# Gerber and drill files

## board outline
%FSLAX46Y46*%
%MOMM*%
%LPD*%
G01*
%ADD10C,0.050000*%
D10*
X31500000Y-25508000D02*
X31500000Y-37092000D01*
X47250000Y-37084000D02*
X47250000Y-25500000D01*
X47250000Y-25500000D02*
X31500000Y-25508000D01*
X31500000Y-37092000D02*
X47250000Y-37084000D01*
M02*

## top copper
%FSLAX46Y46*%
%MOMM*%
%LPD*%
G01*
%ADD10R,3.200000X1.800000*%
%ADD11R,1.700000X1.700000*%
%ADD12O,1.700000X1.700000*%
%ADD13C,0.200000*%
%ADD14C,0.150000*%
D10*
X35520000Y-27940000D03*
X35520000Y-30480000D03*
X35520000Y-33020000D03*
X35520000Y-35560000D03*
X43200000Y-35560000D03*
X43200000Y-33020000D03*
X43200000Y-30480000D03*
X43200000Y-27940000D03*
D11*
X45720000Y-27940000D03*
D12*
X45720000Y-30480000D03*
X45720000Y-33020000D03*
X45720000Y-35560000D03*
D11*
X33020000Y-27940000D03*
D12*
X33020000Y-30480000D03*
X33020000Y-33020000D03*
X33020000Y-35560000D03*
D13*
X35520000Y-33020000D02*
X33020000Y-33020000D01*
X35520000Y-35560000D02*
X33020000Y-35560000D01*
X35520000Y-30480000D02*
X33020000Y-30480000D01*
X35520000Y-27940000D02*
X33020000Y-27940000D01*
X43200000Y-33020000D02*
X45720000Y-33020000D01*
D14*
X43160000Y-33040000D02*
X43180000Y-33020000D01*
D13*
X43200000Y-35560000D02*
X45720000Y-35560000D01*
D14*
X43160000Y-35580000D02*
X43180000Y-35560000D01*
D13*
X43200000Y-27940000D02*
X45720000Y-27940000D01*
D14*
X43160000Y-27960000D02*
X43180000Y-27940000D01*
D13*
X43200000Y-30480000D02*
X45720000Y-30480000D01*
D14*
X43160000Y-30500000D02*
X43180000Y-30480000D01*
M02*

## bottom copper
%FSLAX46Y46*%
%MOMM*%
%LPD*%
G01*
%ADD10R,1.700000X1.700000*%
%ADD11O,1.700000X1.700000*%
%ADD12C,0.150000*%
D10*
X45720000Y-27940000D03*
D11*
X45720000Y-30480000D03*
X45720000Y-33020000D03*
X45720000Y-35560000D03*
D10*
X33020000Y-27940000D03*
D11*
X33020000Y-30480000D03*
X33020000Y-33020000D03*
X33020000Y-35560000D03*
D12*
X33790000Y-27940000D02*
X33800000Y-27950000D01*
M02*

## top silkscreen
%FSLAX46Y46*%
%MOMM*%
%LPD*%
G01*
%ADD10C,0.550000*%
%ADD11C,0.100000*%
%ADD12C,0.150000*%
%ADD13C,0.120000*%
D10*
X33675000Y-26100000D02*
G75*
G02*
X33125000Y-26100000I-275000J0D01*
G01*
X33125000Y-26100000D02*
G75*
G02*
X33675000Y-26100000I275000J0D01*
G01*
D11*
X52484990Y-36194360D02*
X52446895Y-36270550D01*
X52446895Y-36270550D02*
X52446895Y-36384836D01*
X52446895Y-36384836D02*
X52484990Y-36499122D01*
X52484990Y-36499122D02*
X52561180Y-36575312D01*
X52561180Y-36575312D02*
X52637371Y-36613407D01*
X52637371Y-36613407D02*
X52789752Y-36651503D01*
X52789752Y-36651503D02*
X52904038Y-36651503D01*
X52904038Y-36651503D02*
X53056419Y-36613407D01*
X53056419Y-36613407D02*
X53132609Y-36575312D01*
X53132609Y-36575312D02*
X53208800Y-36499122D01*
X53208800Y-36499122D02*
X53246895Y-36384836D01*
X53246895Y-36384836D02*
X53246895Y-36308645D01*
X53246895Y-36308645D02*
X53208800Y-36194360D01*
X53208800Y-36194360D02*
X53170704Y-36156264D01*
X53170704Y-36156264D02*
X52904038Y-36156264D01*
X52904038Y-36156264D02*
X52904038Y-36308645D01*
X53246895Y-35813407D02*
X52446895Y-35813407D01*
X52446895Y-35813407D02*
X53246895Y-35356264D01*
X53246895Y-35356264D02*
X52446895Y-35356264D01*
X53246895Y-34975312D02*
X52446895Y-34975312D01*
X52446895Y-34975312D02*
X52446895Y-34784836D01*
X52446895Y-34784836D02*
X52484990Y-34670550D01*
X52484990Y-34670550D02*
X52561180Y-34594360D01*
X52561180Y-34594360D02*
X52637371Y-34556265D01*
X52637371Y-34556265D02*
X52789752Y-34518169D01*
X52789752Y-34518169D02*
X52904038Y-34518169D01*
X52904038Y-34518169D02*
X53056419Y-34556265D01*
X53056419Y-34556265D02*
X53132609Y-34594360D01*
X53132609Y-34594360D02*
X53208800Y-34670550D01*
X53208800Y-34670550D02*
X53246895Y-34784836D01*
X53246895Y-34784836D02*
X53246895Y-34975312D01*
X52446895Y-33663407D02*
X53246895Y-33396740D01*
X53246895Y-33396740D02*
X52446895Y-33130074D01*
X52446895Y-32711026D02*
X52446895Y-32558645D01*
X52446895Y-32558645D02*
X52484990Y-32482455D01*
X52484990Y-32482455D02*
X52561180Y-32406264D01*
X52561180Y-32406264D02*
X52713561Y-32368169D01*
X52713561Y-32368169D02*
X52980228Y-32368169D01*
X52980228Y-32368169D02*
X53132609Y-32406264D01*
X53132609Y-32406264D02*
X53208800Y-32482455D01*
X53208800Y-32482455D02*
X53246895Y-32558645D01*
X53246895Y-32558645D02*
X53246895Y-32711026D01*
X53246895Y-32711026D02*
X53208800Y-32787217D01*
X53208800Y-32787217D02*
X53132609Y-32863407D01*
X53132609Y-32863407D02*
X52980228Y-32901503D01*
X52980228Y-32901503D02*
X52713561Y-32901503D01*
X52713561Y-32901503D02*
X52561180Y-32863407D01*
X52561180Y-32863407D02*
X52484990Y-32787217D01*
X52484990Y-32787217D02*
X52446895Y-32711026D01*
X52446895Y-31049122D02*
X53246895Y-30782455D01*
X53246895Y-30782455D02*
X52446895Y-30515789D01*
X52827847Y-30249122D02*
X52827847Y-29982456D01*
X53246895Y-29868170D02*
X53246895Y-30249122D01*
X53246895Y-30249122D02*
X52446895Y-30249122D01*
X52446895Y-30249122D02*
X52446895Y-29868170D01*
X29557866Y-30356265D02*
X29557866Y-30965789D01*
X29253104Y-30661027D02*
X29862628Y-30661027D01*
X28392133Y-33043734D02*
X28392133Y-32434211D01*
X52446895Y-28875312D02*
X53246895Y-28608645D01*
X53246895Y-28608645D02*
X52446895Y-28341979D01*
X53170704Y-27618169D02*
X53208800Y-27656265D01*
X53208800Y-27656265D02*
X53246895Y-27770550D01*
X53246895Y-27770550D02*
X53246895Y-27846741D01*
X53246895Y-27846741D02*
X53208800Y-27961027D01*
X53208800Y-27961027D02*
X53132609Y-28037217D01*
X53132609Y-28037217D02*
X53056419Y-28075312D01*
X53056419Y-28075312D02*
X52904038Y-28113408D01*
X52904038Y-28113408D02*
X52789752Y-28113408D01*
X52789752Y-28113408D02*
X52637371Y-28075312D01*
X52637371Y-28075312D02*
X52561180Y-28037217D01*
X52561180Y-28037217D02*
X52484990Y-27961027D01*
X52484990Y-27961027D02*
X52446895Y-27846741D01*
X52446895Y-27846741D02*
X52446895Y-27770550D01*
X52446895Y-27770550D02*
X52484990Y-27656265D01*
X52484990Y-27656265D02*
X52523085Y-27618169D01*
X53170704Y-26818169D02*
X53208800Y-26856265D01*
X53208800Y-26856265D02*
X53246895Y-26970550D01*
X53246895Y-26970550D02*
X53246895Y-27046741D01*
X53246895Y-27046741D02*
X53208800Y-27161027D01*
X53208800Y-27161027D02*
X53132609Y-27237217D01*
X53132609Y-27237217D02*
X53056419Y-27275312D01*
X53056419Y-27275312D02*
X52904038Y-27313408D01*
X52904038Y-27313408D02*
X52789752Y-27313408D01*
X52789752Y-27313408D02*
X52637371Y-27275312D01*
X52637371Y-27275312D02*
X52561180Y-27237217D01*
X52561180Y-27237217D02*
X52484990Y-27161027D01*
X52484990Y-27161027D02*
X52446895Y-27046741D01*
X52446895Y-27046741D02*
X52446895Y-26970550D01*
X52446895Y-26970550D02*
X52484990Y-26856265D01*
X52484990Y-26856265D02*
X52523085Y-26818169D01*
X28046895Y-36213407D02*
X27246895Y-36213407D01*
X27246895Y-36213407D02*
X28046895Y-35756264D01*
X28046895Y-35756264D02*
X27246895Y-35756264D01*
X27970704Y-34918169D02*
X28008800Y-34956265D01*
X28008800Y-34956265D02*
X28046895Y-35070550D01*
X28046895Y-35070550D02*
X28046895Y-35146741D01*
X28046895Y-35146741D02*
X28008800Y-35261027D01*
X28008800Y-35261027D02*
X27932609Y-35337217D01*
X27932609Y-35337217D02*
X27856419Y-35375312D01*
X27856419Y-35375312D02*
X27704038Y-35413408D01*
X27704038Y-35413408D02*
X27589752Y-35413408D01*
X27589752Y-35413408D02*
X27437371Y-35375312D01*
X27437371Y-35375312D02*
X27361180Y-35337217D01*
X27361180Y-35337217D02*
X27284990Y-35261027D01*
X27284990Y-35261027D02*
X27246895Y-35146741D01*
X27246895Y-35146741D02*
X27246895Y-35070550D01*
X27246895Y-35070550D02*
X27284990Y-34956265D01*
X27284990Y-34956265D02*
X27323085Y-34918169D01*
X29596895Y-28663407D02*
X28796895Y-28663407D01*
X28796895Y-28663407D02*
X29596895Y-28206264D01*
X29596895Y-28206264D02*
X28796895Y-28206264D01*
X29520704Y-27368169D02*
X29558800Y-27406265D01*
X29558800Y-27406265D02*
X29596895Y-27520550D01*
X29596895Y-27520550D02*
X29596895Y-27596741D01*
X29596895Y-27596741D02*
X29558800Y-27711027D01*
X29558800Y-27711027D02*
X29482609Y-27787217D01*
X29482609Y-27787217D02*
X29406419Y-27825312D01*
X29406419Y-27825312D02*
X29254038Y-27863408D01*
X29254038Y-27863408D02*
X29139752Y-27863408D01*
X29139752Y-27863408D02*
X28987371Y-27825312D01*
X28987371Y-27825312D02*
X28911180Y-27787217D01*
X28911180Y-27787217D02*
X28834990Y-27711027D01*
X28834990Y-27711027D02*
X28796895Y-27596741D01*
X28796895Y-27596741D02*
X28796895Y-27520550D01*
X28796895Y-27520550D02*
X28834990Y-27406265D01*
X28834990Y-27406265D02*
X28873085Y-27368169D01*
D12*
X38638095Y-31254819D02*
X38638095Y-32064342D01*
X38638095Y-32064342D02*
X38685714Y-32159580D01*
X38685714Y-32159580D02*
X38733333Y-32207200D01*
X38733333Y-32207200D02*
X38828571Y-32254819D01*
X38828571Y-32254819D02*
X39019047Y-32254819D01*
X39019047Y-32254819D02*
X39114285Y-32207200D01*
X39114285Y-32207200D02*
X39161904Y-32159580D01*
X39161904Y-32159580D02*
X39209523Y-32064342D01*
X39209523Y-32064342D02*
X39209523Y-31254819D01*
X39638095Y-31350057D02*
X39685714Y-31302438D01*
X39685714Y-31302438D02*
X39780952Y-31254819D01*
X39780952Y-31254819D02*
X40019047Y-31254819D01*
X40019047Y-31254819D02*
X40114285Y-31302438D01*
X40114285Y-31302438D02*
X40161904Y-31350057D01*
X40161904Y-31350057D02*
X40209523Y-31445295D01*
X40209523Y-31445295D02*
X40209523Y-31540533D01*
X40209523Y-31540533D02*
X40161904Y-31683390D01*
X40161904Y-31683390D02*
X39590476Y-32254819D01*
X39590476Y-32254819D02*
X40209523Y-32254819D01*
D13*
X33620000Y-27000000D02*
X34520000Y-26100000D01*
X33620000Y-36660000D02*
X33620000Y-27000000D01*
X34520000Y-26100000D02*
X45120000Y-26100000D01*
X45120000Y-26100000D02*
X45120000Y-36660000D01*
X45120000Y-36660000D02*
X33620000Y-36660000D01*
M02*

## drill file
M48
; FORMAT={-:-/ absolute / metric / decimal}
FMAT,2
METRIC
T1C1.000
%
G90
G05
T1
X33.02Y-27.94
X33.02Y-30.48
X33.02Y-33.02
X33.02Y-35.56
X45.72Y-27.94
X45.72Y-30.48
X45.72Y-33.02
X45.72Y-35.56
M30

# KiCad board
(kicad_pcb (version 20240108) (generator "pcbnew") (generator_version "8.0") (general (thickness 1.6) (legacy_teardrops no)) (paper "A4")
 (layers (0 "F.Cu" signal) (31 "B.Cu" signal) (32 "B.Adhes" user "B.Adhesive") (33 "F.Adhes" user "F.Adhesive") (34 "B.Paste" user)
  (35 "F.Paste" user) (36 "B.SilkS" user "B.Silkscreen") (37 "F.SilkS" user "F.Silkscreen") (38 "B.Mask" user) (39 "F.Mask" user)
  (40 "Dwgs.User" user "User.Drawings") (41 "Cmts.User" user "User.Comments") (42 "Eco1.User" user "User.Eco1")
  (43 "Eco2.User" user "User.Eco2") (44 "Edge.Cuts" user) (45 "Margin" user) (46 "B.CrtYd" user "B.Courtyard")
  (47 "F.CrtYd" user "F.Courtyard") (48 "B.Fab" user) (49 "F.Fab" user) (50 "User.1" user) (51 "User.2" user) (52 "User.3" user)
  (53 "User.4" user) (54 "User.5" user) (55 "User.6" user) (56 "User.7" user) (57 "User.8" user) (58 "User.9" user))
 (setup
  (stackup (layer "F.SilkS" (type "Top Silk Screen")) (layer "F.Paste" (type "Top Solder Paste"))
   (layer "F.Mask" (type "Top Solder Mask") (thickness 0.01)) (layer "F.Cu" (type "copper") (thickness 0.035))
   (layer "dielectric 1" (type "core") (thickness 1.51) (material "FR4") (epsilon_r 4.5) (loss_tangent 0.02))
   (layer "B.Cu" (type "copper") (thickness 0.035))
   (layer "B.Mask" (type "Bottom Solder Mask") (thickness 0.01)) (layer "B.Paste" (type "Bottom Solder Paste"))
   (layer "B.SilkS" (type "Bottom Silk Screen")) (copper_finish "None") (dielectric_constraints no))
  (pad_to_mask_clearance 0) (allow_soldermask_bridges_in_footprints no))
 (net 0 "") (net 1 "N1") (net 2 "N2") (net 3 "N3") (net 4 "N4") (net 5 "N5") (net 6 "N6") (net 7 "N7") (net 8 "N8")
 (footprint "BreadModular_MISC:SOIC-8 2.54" (layer "F.Cu") (at 38.12 31.75 -90)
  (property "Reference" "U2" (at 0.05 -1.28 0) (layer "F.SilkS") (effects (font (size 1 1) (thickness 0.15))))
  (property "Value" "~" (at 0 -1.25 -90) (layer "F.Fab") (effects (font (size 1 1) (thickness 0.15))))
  (fp_line (start -4.75 4.5) (end -5.65 3.6) (stroke (width 0.12) (type default)) (layer "F.SilkS"))
  (fp_line (start 4.91 4.5) (end -4.75 4.5) (stroke (width 0.12) (type default)) (layer "F.SilkS"))
  (fp_line (start -5.65 3.6) (end -5.65 -7) (stroke (width 0.12) (type default)) (layer "F.SilkS"))
  (fp_line (start -5.65 -7) (end 4.91 -7) (stroke (width 0.12) (type default)) (layer "F.SilkS"))
  (fp_line (start 4.91 -7) (end 4.91 4.5) (stroke (width 0.12) (type default)) (layer "F.SilkS"))
  (pad "1" smd rect (at -3.81 2.6 270) (size 1.8 3.2) (layers "F.Cu" "F.Paste" "F.Mask") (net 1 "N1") (thermal_bridge_angle 45))
  (pad "2" smd rect (at -1.27 2.6 270) (size 1.8 3.2) (layers "F.Cu" "F.Paste" "F.Mask") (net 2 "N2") (thermal_bridge_angle 45))
  (pad "3" smd rect (at 1.27 2.6 270) (size 1.8 3.2) (layers "F.Cu" "F.Paste" "F.Mask") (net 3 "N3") (thermal_bridge_angle 45))
  (pad "4" smd rect (at 3.81 2.6 270) (size 1.8 3.2) (layers "F.Cu" "F.Paste" "F.Mask") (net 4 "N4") (thermal_bridge_angle 45))
  (pad "5" smd rect (at 3.81 -5.08 270) (size 1.8 3.2) (layers "F.Cu" "F.Paste" "F.Mask") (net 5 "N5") (thermal_bridge_angle 45))
  (pad "6" smd rect (at 1.27 -5.08 270) (size 1.8 3.2) (layers "F.Cu" "F.Paste" "F.Mask") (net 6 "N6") (thermal_bridge_angle 45))
  (pad "7" smd rect (at -1.27 -5.08 270) (size 1.8 3.2) (layers "F.Cu" "F.Paste" "F.Mask") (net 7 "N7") (thermal_bridge_angle 45))
  (pad "8" smd rect (at -3.81 -5.08 270) (size 1.8 3.2) (layers "F.Cu" "F.Paste" "F.Mask") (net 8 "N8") (thermal_bridge_angle 45)))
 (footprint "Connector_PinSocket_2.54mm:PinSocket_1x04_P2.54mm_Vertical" (layer "B.Cu") (at 45.72 27.94 180)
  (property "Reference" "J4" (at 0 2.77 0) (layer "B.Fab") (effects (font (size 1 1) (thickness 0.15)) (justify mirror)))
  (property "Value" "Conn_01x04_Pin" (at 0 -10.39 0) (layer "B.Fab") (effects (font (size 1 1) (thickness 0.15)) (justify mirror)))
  (pad "1" thru_hole rect (at 0 0 180) (size 1.7 1.7) (drill 1) (layers "*.Cu" "*.Mask") (remove_unused_layers no) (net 8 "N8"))
  (pad "2" thru_hole oval (at 0 -2.54 180) (size 1.7 1.7) (drill 1) (layers "*.Cu" "*.Mask") (remove_unused_layers no) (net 7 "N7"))
  (pad "3" thru_hole oval (at 0 -5.08 180) (size 1.7 1.7) (drill 1) (layers "*.Cu" "*.Mask") (remove_unused_layers no) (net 6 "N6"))
  (pad "4" thru_hole oval (at 0 -7.62 180) (size 1.7 1.7) (drill 1) (layers "*.Cu" "*.Mask") (remove_unused_layers no) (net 5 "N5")))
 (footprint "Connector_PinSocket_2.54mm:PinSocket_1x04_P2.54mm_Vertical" (layer "B.Cu") (at 33.02 27.94 180)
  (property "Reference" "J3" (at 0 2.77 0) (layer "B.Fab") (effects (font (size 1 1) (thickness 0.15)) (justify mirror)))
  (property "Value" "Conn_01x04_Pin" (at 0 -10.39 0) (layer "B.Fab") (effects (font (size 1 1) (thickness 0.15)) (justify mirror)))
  (pad "1" thru_hole rect (at 0 0 180) (size 1.7 1.7) (drill 1) (layers "*.Cu" "*.Mask") (remove_unused_layers no) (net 1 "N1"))
  (pad "2" thru_hole oval (at 0 -2.54 180) (size 1.7 1.7) (drill 1) (layers "*.Cu" "*.Mask") (remove_unused_layers no) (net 2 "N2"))
  (pad "3" thru_hole oval (at 0 -5.08 180) (size 1.7 1.7) (drill 1) (layers "*.Cu" "*.Mask") (remove_unused_layers no) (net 3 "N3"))
  (pad "4" thru_hole oval (at 0 -7.62 180) (size 1.7 1.7) (drill 1) (layers "*.Cu" "*.Mask") (remove_unused_layers no) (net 4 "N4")))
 (gr_circle (center 33.4 26.1) (end 33.9 26.1) (stroke (width 0.1) (type solid)) (fill solid) (layer "F.SilkS"))
 (gr_line (start 31.5 25.508) (end 31.5 37.092) (stroke (width 0.05) (type default)) (layer "Edge.Cuts"))
 (gr_line (start 47.25 37.084) (end 47.25 25.5) (stroke (width 0.05) (type default)) (layer "Edge.Cuts"))
 (gr_line (start 47.25 25.5) (end 31.5 25.508) (stroke (width 0.05) (type default)) (layer "Edge.Cuts"))
 (gr_line (start 31.5 37.092) (end 47.25 37.084) (stroke (width 0.05) (type default)) (layer "Edge.Cuts"))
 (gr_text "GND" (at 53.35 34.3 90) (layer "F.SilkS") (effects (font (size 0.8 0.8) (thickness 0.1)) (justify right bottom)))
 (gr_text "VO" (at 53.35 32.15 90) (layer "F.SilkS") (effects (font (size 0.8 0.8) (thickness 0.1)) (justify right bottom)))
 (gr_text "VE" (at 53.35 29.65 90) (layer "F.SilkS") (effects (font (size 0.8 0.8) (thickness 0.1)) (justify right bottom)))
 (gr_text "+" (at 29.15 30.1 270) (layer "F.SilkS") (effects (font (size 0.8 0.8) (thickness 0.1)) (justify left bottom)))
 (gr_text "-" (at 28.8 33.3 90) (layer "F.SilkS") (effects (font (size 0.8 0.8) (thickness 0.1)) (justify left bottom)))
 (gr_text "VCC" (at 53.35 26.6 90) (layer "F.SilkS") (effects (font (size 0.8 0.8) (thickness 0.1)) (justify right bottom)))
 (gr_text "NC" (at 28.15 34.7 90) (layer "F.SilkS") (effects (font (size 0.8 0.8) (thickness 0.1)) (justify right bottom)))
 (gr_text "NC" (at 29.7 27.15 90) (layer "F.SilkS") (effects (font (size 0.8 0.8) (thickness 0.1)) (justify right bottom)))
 (segment (start 35.52 33.02) (end 33.02 33.02) (width 0.2) (layer "F.Cu") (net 3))
 (segment (start 35.52 35.56) (end 33.02 35.56) (width 0.2) (layer "F.Cu") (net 4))
 (segment (start 35.52 30.48) (end 33.02 30.48) (width 0.2) (layer "F.Cu") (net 2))
 (segment (start 35.52 27.94) (end 33.02 27.94) (width 0.2) (layer "F.Cu") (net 1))
 (segment (start 33.79 27.94) (end 33.8 27.95) (width 0.15) (layer "B.Cu") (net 1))
 (segment (start 43.2 33.02) (end 45.72 33.02) (width 0.2) (layer "F.Cu") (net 6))
 (segment (start 43.16 33.04) (end 43.18 33.02) (width 0.15) (layer "F.Cu") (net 6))
 (segment (start 43.2 35.56) (end 45.72 35.56) (width 0.2) (layer "F.Cu") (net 5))
 (segment (start 43.16 35.58) (end 43.18 35.56) (width 0.15) (layer "F.Cu") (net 5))
 (segment (start 43.2 27.94) (end 45.72 27.94) (width 0.2) (layer "F.Cu") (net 8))
 (segment (start 43.16 27.96) (end 43.18 27.94) (width 0.15) (layer "F.Cu") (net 8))
 (segment (start 43.2 30.48) (end 45.72 30.48) (width 0.2) (layer "F.Cu") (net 7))
 (segment (start 43.16 30.5) (end 43.18 30.48) (width 0.15) (layer "F.Cu") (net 7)))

